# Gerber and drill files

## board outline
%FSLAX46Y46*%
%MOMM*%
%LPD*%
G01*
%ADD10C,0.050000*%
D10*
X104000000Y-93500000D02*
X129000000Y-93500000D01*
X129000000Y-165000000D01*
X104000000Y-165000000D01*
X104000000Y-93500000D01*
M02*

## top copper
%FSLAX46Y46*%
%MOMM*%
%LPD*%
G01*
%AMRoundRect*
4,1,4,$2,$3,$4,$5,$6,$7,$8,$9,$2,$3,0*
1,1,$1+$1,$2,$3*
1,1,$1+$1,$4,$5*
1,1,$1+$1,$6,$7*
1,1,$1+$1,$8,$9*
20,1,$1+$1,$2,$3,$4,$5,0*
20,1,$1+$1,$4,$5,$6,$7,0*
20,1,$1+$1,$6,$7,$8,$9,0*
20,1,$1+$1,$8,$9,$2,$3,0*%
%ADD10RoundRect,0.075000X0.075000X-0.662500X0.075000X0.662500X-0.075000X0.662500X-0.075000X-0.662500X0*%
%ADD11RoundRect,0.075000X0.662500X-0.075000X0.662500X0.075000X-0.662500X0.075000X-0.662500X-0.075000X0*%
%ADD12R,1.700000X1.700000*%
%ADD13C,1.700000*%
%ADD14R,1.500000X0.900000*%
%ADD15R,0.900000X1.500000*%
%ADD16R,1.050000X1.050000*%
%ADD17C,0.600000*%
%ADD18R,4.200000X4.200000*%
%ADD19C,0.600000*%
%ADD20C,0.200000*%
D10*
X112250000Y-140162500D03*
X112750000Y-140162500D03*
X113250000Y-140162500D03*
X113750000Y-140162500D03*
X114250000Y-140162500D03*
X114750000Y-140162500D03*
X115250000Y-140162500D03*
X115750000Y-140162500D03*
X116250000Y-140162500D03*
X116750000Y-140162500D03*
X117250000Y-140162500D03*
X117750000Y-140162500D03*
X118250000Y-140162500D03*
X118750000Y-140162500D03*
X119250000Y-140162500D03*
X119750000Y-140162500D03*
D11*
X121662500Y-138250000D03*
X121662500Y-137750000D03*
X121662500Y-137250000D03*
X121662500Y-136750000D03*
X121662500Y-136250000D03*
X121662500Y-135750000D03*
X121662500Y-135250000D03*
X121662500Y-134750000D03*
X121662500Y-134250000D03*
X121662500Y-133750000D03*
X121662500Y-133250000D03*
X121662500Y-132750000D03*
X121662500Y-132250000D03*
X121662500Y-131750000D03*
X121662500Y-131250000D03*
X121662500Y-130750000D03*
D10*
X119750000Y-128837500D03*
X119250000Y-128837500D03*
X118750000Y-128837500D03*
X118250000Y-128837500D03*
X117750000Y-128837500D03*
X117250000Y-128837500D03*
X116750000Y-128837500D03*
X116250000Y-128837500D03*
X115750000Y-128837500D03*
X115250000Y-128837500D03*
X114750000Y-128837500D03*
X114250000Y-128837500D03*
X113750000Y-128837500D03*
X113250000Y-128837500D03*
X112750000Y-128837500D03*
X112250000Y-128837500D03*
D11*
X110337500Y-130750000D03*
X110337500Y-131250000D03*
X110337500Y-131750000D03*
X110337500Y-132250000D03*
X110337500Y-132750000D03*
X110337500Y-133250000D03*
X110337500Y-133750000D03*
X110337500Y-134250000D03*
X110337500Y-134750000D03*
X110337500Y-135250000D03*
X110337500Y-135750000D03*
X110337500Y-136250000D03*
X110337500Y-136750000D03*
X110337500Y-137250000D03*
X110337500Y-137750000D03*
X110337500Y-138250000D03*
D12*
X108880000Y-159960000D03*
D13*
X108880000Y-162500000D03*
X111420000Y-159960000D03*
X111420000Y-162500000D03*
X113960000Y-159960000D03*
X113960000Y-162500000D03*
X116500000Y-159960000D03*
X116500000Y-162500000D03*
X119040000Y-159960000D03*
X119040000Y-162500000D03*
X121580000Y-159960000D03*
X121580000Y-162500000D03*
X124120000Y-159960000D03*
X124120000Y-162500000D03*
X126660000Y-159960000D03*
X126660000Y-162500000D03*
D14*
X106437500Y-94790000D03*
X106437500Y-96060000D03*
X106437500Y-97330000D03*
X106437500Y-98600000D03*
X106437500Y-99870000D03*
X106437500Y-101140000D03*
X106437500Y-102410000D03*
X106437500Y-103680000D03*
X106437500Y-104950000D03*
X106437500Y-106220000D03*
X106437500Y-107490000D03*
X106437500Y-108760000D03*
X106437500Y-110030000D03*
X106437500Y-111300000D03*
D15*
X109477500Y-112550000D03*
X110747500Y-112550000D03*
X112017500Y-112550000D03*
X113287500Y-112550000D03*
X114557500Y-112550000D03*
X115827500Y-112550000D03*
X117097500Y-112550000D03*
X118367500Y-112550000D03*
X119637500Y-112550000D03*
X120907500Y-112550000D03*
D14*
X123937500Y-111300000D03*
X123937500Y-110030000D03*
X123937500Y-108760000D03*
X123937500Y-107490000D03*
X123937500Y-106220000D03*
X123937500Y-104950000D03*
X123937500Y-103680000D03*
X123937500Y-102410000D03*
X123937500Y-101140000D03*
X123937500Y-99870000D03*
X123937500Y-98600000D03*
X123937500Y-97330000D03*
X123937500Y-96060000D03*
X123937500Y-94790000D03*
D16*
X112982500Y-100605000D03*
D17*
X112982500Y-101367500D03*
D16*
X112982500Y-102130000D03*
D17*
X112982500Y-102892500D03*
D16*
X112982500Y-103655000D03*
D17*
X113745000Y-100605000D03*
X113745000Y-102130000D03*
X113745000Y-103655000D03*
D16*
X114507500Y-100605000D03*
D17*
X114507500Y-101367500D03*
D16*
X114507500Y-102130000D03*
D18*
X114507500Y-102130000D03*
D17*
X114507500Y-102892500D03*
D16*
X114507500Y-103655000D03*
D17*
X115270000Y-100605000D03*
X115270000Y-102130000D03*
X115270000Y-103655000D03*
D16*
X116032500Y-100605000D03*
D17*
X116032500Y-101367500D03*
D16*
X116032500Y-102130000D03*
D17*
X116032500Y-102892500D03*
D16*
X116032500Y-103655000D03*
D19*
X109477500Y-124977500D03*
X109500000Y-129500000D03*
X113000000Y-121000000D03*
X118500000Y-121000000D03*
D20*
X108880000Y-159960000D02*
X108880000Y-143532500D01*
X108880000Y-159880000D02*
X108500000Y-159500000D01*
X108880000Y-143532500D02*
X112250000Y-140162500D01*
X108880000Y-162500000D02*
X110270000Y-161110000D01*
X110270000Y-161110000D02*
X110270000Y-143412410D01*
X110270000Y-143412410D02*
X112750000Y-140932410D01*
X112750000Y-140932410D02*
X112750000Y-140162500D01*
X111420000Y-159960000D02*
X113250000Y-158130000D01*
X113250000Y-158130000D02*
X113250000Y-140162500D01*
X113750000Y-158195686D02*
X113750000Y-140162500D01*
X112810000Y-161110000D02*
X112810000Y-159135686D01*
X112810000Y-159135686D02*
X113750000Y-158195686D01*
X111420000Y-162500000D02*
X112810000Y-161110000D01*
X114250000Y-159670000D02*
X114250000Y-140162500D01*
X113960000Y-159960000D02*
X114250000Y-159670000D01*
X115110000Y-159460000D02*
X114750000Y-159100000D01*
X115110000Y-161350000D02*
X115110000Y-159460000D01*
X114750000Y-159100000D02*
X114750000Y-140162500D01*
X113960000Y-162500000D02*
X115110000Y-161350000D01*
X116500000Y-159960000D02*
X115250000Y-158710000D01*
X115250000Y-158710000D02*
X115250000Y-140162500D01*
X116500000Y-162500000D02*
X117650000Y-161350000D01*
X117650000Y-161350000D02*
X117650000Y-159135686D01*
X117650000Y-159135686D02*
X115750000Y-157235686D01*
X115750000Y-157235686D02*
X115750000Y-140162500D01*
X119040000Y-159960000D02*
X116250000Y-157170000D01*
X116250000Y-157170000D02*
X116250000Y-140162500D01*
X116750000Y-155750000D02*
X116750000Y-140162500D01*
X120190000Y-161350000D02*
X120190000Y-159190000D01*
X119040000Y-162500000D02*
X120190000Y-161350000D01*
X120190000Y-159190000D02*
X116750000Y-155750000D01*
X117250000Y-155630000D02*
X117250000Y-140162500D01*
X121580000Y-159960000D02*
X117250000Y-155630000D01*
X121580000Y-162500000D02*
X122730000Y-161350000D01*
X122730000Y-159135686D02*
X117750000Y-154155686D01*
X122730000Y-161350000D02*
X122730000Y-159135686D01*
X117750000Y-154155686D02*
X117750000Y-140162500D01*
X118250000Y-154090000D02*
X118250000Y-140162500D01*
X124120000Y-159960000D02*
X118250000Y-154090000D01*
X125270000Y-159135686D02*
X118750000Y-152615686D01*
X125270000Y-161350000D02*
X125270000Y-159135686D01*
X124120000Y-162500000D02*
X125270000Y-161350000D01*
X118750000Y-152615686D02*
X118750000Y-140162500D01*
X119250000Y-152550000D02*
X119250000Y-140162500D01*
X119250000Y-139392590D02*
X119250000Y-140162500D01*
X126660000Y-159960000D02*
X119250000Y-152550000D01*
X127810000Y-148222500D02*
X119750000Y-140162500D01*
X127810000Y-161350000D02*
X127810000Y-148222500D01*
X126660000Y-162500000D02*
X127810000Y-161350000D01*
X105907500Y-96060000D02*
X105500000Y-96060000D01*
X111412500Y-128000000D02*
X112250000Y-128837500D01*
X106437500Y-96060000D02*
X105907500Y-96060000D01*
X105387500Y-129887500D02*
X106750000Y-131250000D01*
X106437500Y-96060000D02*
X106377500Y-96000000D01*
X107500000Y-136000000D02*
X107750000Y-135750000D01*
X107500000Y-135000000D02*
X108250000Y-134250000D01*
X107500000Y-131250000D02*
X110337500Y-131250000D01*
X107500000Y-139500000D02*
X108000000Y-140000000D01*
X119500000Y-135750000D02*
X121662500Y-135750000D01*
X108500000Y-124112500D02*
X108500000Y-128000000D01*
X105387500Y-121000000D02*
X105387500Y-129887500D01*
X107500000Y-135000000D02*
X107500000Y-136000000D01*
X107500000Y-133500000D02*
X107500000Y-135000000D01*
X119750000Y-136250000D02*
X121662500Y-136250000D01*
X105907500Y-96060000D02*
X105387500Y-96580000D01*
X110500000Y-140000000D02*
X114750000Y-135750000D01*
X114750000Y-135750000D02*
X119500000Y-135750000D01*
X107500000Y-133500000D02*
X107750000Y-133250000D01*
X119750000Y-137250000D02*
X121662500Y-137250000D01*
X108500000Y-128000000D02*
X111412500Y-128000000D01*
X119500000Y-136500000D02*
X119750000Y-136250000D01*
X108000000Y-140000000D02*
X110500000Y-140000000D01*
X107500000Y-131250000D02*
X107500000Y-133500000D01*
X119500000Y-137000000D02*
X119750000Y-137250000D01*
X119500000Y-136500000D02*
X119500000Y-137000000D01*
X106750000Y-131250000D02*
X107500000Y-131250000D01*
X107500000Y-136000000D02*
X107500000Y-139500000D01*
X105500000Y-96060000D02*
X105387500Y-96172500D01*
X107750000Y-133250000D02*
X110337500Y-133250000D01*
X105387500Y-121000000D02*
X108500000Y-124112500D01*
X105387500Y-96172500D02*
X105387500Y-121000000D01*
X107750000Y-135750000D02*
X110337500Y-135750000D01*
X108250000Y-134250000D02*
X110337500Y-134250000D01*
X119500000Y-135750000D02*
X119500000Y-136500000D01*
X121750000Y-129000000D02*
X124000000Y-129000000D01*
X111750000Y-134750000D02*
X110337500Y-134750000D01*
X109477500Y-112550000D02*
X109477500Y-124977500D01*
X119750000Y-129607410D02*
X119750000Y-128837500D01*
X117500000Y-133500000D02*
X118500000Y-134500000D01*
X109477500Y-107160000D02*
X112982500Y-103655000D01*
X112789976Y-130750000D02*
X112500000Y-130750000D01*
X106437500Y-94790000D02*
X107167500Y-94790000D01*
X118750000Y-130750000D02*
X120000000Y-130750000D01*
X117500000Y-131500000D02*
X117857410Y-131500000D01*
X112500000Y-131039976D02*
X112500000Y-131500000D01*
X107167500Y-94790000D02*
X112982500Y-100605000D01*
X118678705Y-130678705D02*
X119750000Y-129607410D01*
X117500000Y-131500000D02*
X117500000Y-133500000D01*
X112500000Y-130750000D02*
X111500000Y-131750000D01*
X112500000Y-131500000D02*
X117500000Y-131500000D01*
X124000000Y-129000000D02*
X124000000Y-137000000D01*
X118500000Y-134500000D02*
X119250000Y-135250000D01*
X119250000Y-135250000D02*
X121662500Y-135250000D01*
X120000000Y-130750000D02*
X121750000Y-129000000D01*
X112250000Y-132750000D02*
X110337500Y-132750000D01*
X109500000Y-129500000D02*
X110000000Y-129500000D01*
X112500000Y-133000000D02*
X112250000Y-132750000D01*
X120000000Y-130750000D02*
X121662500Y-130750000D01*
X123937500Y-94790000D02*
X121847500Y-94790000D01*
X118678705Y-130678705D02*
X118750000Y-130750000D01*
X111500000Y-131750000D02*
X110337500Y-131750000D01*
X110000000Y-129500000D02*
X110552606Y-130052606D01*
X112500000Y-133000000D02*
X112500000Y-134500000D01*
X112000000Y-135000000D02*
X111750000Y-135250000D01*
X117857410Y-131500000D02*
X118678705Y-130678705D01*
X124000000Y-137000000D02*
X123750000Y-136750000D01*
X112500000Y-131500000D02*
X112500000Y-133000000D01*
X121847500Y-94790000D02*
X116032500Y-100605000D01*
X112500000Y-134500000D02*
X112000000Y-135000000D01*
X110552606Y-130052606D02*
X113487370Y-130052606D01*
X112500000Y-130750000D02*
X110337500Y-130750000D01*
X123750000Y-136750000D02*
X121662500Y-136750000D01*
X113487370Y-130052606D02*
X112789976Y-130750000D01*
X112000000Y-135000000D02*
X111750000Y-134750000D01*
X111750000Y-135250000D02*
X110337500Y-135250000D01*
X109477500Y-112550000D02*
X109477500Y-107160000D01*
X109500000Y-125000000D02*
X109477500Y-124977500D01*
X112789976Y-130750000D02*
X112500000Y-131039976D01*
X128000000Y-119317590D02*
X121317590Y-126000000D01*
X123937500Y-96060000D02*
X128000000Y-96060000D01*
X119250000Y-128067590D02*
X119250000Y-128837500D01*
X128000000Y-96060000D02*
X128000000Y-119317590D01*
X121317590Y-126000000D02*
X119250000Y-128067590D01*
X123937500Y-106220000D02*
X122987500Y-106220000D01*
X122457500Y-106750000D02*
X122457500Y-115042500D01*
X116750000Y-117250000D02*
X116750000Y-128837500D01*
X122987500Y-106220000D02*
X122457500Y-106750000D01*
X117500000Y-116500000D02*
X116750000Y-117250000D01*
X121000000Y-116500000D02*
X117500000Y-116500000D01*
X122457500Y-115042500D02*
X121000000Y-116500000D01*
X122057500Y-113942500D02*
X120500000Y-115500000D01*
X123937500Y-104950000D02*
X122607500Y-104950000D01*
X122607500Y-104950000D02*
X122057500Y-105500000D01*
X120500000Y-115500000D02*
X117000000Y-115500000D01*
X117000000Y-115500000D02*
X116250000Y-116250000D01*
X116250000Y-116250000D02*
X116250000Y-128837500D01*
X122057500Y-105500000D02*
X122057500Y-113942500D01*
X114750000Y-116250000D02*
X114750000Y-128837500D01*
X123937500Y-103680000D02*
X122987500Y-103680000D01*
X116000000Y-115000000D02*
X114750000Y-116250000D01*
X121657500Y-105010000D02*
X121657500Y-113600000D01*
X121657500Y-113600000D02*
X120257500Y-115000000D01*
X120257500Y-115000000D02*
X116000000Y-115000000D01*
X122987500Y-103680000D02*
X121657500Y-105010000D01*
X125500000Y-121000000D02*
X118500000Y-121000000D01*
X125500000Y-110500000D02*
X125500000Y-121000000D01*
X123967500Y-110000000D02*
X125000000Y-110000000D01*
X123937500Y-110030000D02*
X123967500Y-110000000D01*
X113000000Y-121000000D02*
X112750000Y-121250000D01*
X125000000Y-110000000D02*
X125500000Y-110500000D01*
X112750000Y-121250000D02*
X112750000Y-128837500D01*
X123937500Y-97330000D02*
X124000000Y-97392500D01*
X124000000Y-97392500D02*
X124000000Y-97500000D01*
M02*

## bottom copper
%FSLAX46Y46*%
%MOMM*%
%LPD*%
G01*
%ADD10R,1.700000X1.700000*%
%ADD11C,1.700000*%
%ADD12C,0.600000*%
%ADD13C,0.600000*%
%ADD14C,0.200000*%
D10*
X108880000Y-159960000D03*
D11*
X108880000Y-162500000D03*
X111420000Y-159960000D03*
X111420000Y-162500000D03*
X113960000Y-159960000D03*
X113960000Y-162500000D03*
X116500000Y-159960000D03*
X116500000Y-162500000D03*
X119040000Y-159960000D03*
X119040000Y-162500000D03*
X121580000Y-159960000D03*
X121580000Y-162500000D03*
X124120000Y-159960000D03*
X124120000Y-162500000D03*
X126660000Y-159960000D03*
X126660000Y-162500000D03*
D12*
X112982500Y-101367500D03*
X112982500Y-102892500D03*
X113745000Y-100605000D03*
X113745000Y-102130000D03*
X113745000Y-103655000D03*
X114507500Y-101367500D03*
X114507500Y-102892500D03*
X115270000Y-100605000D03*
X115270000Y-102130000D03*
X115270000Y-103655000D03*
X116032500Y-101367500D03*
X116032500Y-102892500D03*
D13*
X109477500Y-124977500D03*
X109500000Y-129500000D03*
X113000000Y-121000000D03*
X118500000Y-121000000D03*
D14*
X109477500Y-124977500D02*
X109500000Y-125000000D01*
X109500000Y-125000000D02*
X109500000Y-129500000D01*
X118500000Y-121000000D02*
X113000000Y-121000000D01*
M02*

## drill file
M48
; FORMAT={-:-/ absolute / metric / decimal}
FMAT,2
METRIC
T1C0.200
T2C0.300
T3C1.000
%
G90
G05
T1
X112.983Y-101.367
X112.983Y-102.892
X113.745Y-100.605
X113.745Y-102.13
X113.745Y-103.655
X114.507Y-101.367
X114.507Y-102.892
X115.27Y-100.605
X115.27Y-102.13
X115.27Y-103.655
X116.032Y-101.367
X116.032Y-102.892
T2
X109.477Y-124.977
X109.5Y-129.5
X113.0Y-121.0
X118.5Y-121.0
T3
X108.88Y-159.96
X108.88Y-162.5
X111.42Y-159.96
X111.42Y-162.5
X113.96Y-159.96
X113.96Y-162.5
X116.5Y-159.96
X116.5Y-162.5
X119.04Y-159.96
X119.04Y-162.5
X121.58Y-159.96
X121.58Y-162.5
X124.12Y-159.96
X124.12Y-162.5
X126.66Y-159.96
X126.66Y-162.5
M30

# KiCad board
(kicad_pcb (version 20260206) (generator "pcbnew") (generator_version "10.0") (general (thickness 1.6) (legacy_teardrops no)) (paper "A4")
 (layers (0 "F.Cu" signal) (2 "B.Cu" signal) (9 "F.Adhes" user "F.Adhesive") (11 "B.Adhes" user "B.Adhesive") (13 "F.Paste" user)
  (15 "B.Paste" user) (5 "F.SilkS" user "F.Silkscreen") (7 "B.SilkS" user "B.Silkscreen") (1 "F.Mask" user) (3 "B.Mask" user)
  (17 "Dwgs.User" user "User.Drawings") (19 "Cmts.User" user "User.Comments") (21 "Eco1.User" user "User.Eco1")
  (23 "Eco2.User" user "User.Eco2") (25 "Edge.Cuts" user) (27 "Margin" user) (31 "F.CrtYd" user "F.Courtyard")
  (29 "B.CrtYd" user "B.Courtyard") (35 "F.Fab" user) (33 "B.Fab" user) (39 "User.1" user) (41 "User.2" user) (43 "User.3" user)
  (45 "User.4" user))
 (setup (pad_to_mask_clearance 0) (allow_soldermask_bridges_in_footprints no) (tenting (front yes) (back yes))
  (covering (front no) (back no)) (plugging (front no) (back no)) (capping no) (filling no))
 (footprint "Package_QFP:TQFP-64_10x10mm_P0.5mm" (layer "F.Cu") (at 116 134.5 90)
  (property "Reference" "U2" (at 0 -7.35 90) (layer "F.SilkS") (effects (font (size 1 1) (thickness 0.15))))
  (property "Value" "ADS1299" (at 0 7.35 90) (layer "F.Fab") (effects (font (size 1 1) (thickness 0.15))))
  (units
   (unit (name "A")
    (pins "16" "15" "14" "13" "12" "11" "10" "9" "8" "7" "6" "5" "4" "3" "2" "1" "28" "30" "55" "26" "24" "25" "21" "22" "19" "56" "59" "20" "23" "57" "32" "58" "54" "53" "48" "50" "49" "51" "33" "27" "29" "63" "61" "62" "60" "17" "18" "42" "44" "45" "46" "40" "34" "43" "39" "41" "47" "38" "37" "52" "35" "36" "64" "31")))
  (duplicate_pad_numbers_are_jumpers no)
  (pad "1" smd roundrect (at -5.6625 -3.75 90) (size 1.475 0.3) (layers "F.Cu" "F.Mask" "F.Paste") (roundrect_rratio 0.25)
   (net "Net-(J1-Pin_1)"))
  (pad "2" smd roundrect (at -5.6625 -3.25 90) (size 1.475 0.3) (layers "F.Cu" "F.Mask" "F.Paste") (roundrect_rratio 0.25)
   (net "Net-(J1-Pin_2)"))
  (pad "3" smd roundrect (at -5.6625 -2.75 90) (size 1.475 0.3) (layers "F.Cu" "F.Mask" "F.Paste") (roundrect_rratio 0.25)
   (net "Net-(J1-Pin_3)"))
  (pad "4" smd roundrect (at -5.6625 -2.25 90) (size 1.475 0.3) (layers "F.Cu" "F.Mask" "F.Paste") (roundrect_rratio 0.25)
   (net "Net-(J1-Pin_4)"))
  (pad "5" smd roundrect (at -5.6625 -1.75 90) (size 1.475 0.3) (layers "F.Cu" "F.Mask" "F.Paste") (roundrect_rratio 0.25)
   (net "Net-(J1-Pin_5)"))
  (pad "6" smd roundrect (at -5.6625 -1.25 90) (size 1.475 0.3) (layers "F.Cu" "F.Mask" "F.Paste") (roundrect_rratio 0.25)
   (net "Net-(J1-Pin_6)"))
  (pad "7" smd roundrect (at -5.6625 -0.75 90) (size 1.475 0.3) (layers "F.Cu" "F.Mask" "F.Paste") (roundrect_rratio 0.25)
   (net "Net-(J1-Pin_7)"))
  (pad "8" smd roundrect (at -5.6625 -0.25 90) (size 1.475 0.3) (layers "F.Cu" "F.Mask" "F.Paste") (roundrect_rratio 0.25)
   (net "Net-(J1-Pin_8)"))
  (pad "9" smd roundrect (at -5.6625 0.25 90) (size 1.475 0.3) (layers "F.Cu" "F.Mask" "F.Paste") (roundrect_rratio 0.25)
   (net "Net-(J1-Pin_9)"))
  (pad "10" smd roundrect (at -5.6625 0.75 90) (size 1.475 0.3) (layers "F.Cu" "F.Mask" "F.Paste") (roundrect_rratio 0.25)
   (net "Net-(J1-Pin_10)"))
  (pad "11" smd roundrect (at -5.6625 1.25 90) (size 1.475 0.3) (layers "F.Cu" "F.Mask" "F.Paste") (roundrect_rratio 0.25)
   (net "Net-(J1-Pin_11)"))
  (pad "12" smd roundrect (at -5.6625 1.75 90) (size 1.475 0.3) (layers "F.Cu" "F.Mask" "F.Paste") (roundrect_rratio 0.25)
   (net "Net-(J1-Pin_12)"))
  (pad "13" smd roundrect (at -5.6625 2.25 90) (size 1.475 0.3) (layers "F.Cu" "F.Mask" "F.Paste") (roundrect_rratio 0.25)
   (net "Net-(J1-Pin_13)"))
  (pad "14" smd roundrect (at -5.6625 2.75 90) (size 1.475 0.3) (layers "F.Cu" "F.Mask" "F.Paste") (roundrect_rratio 0.25)
   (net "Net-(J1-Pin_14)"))
  (pad "15" smd roundrect (at -5.6625 3.25 90) (size 1.475 0.3) (layers "F.Cu" "F.Mask" "F.Paste") (roundrect_rratio 0.25)
   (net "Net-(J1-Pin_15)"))
  (pad "16" smd roundrect (at -5.6625 3.75 90) (size 1.475 0.3) (layers "F.Cu" "F.Mask" "F.Paste") (roundrect_rratio 0.25)
   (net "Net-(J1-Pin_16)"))
  (pad "17" smd roundrect (at -3.75 5.6625 90) (size 0.3 1.475) (layers "F.Cu" "F.Mask" "F.Paste") (roundrect_rratio 0.25)
   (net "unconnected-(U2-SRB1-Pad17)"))
  (pad "18" smd roundrect (at -3.25 5.6625 90) (size 0.3 1.475) (layers "F.Cu" "F.Mask" "F.Paste") (roundrect_rratio 0.25)
   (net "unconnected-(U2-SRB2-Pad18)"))
  (pad "19" smd roundrect (at -2.75 5.6625 90) (size 0.3 1.475) (layers "F.Cu" "F.Mask" "F.Paste") (roundrect_rratio 0.25) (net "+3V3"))
  (pad "20" smd roundrect (at -2.25 5.6625 90) (size 0.3 1.475) (layers "F.Cu" "F.Mask" "F.Paste") (roundrect_rratio 0.25) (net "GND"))
  (pad "21" smd roundrect (at -1.75 5.6625 90) (size 0.3 1.475) (layers "F.Cu" "F.Mask" "F.Paste") (roundrect_rratio 0.25) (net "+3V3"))
  (pad "22" smd roundrect (at -1.25 5.6625 90) (size 0.3 1.475) (layers "F.Cu" "F.Mask" "F.Paste") (roundrect_rratio 0.25) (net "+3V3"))
  (pad "23" smd roundrect (at -0.75 5.6625 90) (size 0.3 1.475) (layers "F.Cu" "F.Mask" "F.Paste") (roundrect_rratio 0.25) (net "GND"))
  (pad "24" smd roundrect (at -0.25 5.6625 90) (size 0.3 1.475) (layers "F.Cu" "F.Mask" "F.Paste") (roundrect_rratio 0.25)
   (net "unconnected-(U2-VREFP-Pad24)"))
  (pad "25" smd roundrect (at 0.25 5.6625 90) (size 0.3 1.475) (layers "F.Cu" "F.Mask" "F.Paste") (roundrect_rratio 0.25)
   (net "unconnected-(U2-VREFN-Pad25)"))
  (pad "26" smd roundrect (at 0.75 5.6625 90) (size 0.3 1.475) (layers "F.Cu" "F.Mask" "F.Paste") (roundrect_rratio 0.25)
   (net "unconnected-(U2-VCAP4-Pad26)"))
  (pad "27" smd roundrect (at 1.25 5.6625 90) (size 0.3 1.475) (layers "F.Cu" "F.Mask" "F.Paste") (roundrect_rratio 0.25)
   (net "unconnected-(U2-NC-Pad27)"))
  (pad "28" smd roundrect (at 1.75 5.6625 90) (size 0.3 1.475) (layers "F.Cu" "F.Mask" "F.Paste") (roundrect_rratio 0.25)
   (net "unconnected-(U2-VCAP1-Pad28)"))
  (pad "29" smd roundrect (at 2.25 5.6625 90) (size 0.3 1.475) (layers "F.Cu" "F.Mask" "F.Paste") (roundrect_rratio 0.25)
   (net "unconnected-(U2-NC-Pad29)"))
  (pad "30" smd roundrect (at 2.75 5.6625 90) (size 0.3 1.475) (layers "F.Cu" "F.Mask" "F.Paste") (roundrect_rratio 0.25)
   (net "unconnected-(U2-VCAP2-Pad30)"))
  (pad "31" smd roundrect (at 3.25 5.6625 90) (size 0.3 1.475) (layers "F.Cu" "F.Mask" "F.Paste") (roundrect_rratio 0.25)
   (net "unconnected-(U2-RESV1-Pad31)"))
  (pad "32" smd roundrect (at 3.75 5.6625 90) (size 0.3 1.475) (layers "F.Cu" "F.Mask" "F.Paste") (roundrect_rratio 0.25) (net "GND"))
  (pad "33" smd roundrect (at 5.6625 3.75 90) (size 1.475 0.3) (layers "F.Cu" "F.Mask" "F.Paste") (roundrect_rratio 0.25) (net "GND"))
  (pad "34" smd roundrect (at 5.6625 3.25 90) (size 1.475 0.3) (layers "F.Cu" "F.Mask" "F.Paste") (roundrect_rratio 0.25)
   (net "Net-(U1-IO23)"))
  (pad "35" smd roundrect (at 5.6625 2.75 90) (size 1.475 0.3) (layers "F.Cu" "F.Mask" "F.Paste") (roundrect_rratio 0.25)
   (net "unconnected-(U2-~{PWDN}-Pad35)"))
  (pad "36" smd roundrect (at 5.6625 2.25 90) (size 1.475 0.3) (layers "F.Cu" "F.Mask" "F.Paste") (roundrect_rratio 0.25)
   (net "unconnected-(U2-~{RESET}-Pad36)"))
  (pad "37" smd roundrect (at 5.6625 1.75 90) (size 1.475 0.3) (layers "F.Cu" "F.Mask" "F.Paste") (roundrect_rratio 0.25)
   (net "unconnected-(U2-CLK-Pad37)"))
  (pad "38" smd roundrect (at 5.6625 1.25 90) (size 1.475 0.3) (layers "F.Cu" "F.Mask" "F.Paste") (roundrect_rratio 0.25)
   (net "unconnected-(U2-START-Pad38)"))
  (pad "39" smd roundrect (at 5.6625 0.75 90) (size 1.475 0.3) (layers "F.Cu" "F.Mask" "F.Paste") (roundrect_rratio 0.25)
   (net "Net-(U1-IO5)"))
  (pad "40" smd roundrect (at 5.6625 0.25 90) (size 1.475 0.3) (layers "F.Cu" "F.Mask" "F.Paste") (roundrect_rratio 0.25)
   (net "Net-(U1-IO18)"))
  (pad "41" smd roundrect (at 5.6625 -0.25 90) (size 1.475 0.3) (layers "F.Cu" "F.Mask" "F.Paste") (roundrect_rratio 0.25)
   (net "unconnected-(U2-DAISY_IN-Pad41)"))
  (pad "42" smd roundrect (at 5.6625 -0.75 90) (size 1.475 0.3) (layers "F.Cu" "F.Mask" "F.Paste") (roundrect_rratio 0.25)
   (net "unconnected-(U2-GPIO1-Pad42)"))
  (pad "43" smd roundrect (at 5.6625 -1.25 90) (size 1.475 0.3) (layers "F.Cu" "F.Mask" "F.Paste") (roundrect_rratio 0.25)
   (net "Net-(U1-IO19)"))
  (pad "44" smd roundrect (at 5.6625 -1.75 90) (size 1.475 0.3) (layers "F.Cu" "F.Mask" "F.Paste") (roundrect_rratio 0.25)
   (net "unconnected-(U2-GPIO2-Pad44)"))
  (pad "45" smd roundrect (at 5.6625 -2.25 90) (size 1.475 0.3) (layers "F.Cu" "F.Mask" "F.Paste") (roundrect_rratio 0.25)
   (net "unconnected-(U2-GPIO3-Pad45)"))
  (pad "46" smd roundrect (at 5.6625 -2.75 90) (size 1.475 0.3) (layers "F.Cu" "F.Mask" "F.Paste") (roundrect_rratio 0.25)
   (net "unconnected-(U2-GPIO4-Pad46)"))
  (pad "47" smd roundrect (at 5.6625 -3.25 90) (size 1.475 0.3) (layers "F.Cu" "F.Mask" "F.Paste") (roundrect_rratio 0.25)
   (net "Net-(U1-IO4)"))
  (pad "48" smd roundrect (at 5.6625 -3.75 90) (size 1.475 0.3) (layers "F.Cu" "F.Mask" "F.Paste") (roundrect_rratio 0.25) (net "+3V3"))
  (pad "49" smd roundrect (at 3.75 -5.6625 90) (size 0.3 1.475) (layers "F.Cu" "F.Mask" "F.Paste") (roundrect_rratio 0.25) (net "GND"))
  (pad "50" smd roundrect (at 3.25 -5.6625 90) (size 0.3 1.475) (layers "F.Cu" "F.Mask" "F.Paste") (roundrect_rratio 0.25) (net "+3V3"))
  (pad "51" smd roundrect (at 2.75 -5.6625 90) (size 0.3 1.475) (layers "F.Cu" "F.Mask" "F.Paste") (roundrect_rratio 0.25) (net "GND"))
  (pad "52" smd roundrect (at 2.25 -5.6625 90) (size 0.3 1.475) (layers "F.Cu" "F.Mask" "F.Paste") (roundrect_rratio 0.25)
   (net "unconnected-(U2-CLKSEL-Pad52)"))
  (pad "53" smd roundrect (at 1.75 -5.6625 90) (size 0.3 1.475) (layers "F.Cu" "F.Mask" "F.Paste") (roundrect_rratio 0.25) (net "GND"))
  (pad "54" smd roundrect (at 1.25 -5.6625 90) (size 0.3 1.475) (layers "F.Cu" "F.Mask" "F.Paste") (roundrect_rratio 0.25) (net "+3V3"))
  (pad "55" smd roundrect (at 0.75 -5.6625 90) (size 0.3 1.475) (layers "F.Cu" "F.Mask" "F.Paste") (roundrect_rratio 0.25)
   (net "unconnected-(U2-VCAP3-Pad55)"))
  (pad "56" smd roundrect (at 0.25 -5.6625 90) (size 0.3 1.475) (layers "F.Cu" "F.Mask" "F.Paste") (roundrect_rratio 0.25) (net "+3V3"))
  (pad "57" smd roundrect (at -0.25 -5.6625 90) (size 0.3 1.475) (layers "F.Cu" "F.Mask" "F.Paste") (roundrect_rratio 0.25) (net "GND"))
  (pad "58" smd roundrect (at -0.75 -5.6625 90) (size 0.3 1.475) (layers "F.Cu" "F.Mask" "F.Paste") (roundrect_rratio 0.25) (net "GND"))
  (pad "59" smd roundrect (at -1.25 -5.6625 90) (size 0.3 1.475) (layers "F.Cu" "F.Mask" "F.Paste") (roundrect_rratio 0.25) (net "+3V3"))
  (pad "60" smd roundrect (at -1.75 -5.6625 90) (size 0.3 1.475) (layers "F.Cu" "F.Mask" "F.Paste") (roundrect_rratio 0.25)
   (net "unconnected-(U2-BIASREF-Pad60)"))
  (pad "61" smd roundrect (at -2.25 -5.6625 90) (size 0.3 1.475) (layers "F.Cu" "F.Mask" "F.Paste") (roundrect_rratio 0.25)
   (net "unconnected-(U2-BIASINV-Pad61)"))
  (pad "62" smd roundrect (at -2.75 -5.6625 90) (size 0.3 1.475) (layers "F.Cu" "F.Mask" "F.Paste") (roundrect_rratio 0.25)
   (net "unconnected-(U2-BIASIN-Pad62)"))
  (pad "63" smd roundrect (at -3.25 -5.6625 90) (size 0.3 1.475) (layers "F.Cu" "F.Mask" "F.Paste") (roundrect_rratio 0.25)
   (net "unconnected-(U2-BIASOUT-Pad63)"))
  (pad "64" smd roundrect (at -3.75 -5.6625 90) (size 0.3 1.475) (layers "F.Cu" "F.Mask" "F.Paste") (roundrect_rratio 0.25)
   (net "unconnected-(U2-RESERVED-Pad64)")))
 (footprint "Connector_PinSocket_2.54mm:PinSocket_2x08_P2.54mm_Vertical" (layer "F.Cu") (at 108.88 159.96 90)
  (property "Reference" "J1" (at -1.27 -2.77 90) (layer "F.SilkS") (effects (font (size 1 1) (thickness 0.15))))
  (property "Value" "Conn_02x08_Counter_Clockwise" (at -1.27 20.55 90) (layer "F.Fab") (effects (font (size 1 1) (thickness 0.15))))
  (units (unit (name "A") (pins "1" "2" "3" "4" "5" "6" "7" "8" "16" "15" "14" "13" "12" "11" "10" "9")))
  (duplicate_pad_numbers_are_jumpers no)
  (pad "1" thru_hole rect (at 0 0 90) (size 1.7 1.7) (drill 1) (layers "*.Cu" "*.Mask") (remove_unused_layers no) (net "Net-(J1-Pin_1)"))
  (pad "2" thru_hole circle (at -2.54 0 90) (size 1.7 1.7) (drill 1) (layers "*.Cu" "*.Mask") (remove_unused_layers no)
   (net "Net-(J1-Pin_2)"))
  (pad "3" thru_hole circle (at 0 2.54 90) (size 1.7 1.7) (drill 1) (layers "*.Cu" "*.Mask") (remove_unused_layers no)
   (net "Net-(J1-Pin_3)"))
  (pad "4" thru_hole circle (at -2.54 2.54 90) (size 1.7 1.7) (drill 1) (layers "*.Cu" "*.Mask") (remove_unused_layers no)
   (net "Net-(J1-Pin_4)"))
  (pad "5" thru_hole circle (at 0 5.08 90) (size 1.7 1.7) (drill 1) (layers "*.Cu" "*.Mask") (remove_unused_layers no)
   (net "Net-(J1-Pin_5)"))
  (pad "6" thru_hole circle (at -2.54 5.08 90) (size 1.7 1.7) (drill 1) (layers "*.Cu" "*.Mask") (remove_unused_layers no)
   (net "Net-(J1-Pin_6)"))
  (pad "7" thru_hole circle (at 0 7.62 90) (size 1.7 1.7) (drill 1) (layers "*.Cu" "*.Mask") (remove_unused_layers no)
   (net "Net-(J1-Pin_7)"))
  (pad "8" thru_hole circle (at -2.54 7.62 90) (size 1.7 1.7) (drill 1) (layers "*.Cu" "*.Mask") (remove_unused_layers no)
   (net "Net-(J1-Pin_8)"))
  (pad "9" thru_hole circle (at 0 10.16 90) (size 1.7 1.7) (drill 1) (layers "*.Cu" "*.Mask") (remove_unused_layers no)
   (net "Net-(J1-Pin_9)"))
  (pad "10" thru_hole circle (at -2.54 10.16 90) (size 1.7 1.7) (drill 1) (layers "*.Cu" "*.Mask") (remove_unused_layers no)
   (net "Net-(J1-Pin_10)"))
  (pad "11" thru_hole circle (at 0 12.7 90) (size 1.7 1.7) (drill 1) (layers "*.Cu" "*.Mask") (remove_unused_layers no)
   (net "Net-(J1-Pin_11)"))
  (pad "12" thru_hole circle (at -2.54 12.7 90) (size 1.7 1.7) (drill 1) (layers "*.Cu" "*.Mask") (remove_unused_layers no)
   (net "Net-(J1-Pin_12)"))
  (pad "13" thru_hole circle (at 0 15.24 90) (size 1.7 1.7) (drill 1) (layers "*.Cu" "*.Mask") (remove_unused_layers no)
   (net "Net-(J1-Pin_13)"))
  (pad "14" thru_hole circle (at -2.54 15.24 90) (size 1.7 1.7) (drill 1) (layers "*.Cu" "*.Mask") (remove_unused_layers no)
   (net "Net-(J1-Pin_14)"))
  (pad "15" thru_hole circle (at 0 17.78 90) (size 1.7 1.7) (drill 1) (layers "*.Cu" "*.Mask") (remove_unused_layers no)
   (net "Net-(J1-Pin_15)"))
  (pad "16" thru_hole circle (at -2.54 17.78 90) (size 1.7 1.7) (drill 1) (layers "*.Cu" "*.Mask") (remove_unused_layers no)
   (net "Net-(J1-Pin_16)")))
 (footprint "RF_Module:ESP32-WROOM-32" (layer "F.Cu") (at 115.1875 103.04)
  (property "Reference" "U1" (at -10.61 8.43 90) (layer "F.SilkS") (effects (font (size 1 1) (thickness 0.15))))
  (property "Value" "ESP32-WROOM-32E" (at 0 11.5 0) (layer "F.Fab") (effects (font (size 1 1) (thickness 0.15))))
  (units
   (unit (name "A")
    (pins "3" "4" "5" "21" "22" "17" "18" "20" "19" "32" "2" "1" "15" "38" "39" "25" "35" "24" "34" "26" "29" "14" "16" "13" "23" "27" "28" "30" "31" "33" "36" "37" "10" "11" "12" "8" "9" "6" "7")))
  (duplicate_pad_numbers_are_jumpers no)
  (pad "1" smd rect (at -8.75 -8.25) (size 1.5 0.9) (layers "F.Cu" "F.Mask" "F.Paste") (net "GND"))
  (pad "2" smd rect (at -8.75 -6.98) (size 1.5 0.9) (layers "F.Cu" "F.Mask" "F.Paste") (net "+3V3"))
  (pad "3" smd rect (at -8.75 -5.71) (size 1.5 0.9) (layers "F.Cu" "F.Mask" "F.Paste") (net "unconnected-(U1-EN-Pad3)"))
  (pad "4" smd rect (at -8.75 -4.44) (size 1.5 0.9) (layers "F.Cu" "F.Mask" "F.Paste") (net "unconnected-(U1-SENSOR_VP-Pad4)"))
  (pad "5" smd rect (at -8.75 -3.17) (size 1.5 0.9) (layers "F.Cu" "F.Mask" "F.Paste") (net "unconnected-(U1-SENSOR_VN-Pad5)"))
  (pad "6" smd rect (at -8.75 -1.9) (size 1.5 0.9) (layers "F.Cu" "F.Mask" "F.Paste") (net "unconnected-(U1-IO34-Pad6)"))
  (pad "7" smd rect (at -8.75 -0.63) (size 1.5 0.9) (layers "F.Cu" "F.Mask" "F.Paste") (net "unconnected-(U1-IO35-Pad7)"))
  (pad "8" smd rect (at -8.75 0.64) (size 1.5 0.9) (layers "F.Cu" "F.Mask" "F.Paste") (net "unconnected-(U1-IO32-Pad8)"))
  (pad "9" smd rect (at -8.75 1.91) (size 1.5 0.9) (layers "F.Cu" "F.Mask" "F.Paste") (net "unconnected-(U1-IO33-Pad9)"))
  (pad "10" smd rect (at -8.75 3.18) (size 1.5 0.9) (layers "F.Cu" "F.Mask" "F.Paste") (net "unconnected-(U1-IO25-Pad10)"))
  (pad "11" smd rect (at -8.75 4.45) (size 1.5 0.9) (layers "F.Cu" "F.Mask" "F.Paste") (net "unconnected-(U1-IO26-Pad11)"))
  (pad "12" smd rect (at -8.75 5.72) (size 1.5 0.9) (layers "F.Cu" "F.Mask" "F.Paste") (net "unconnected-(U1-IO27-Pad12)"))
  (pad "13" smd rect (at -8.75 6.99) (size 1.5 0.9) (layers "F.Cu" "F.Mask" "F.Paste") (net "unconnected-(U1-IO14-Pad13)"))
  (pad "14" smd rect (at -8.75 8.26) (size 1.5 0.9) (layers "F.Cu" "F.Mask" "F.Paste") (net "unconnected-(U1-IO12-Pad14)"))
  (pad "15" smd rect (at -5.71 9.51 90) (size 1.5 0.9) (layers "F.Cu" "F.Mask" "F.Paste") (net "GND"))
  (pad "16" smd rect (at -4.44 9.51 90) (size 1.5 0.9) (layers "F.Cu" "F.Mask" "F.Paste") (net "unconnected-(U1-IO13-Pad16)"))
  (pad "17" smd rect (at -3.17 9.51 90) (size 1.5 0.9) (layers "F.Cu" "F.Mask" "F.Paste") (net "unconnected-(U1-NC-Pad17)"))
  (pad "18" smd rect (at -1.9 9.51 90) (size 1.5 0.9) (layers "F.Cu" "F.Mask" "F.Paste") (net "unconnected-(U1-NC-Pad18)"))
  (pad "19" smd rect (at -0.63 9.51 90) (size 1.5 0.9) (layers "F.Cu" "F.Mask" "F.Paste") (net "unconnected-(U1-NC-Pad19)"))
  (pad "20" smd rect (at 0.64 9.51 90) (size 1.5 0.9) (layers "F.Cu" "F.Mask" "F.Paste") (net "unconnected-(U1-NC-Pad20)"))
  (pad "21" smd rect (at 1.91 9.51 90) (size 1.5 0.9) (layers "F.Cu" "F.Mask" "F.Paste") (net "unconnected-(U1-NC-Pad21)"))
  (pad "22" smd rect (at 3.18 9.51 90) (size 1.5 0.9) (layers "F.Cu" "F.Mask" "F.Paste") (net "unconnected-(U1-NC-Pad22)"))
  (pad "23" smd rect (at 4.45 9.51 90) (size 1.5 0.9) (layers "F.Cu" "F.Mask" "F.Paste") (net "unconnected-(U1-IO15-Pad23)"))
  (pad "24" smd rect (at 5.72 9.51 90) (size 1.5 0.9) (layers "F.Cu" "F.Mask" "F.Paste") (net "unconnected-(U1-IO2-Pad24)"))
  (pad "25" smd rect (at 8.75 8.26) (size 1.5 0.9) (layers "F.Cu" "F.Mask" "F.Paste") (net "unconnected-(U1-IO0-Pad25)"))
  (pad "26" smd rect (at 8.75 6.99) (size 1.5 0.9) (layers "F.Cu" "F.Mask" "F.Paste") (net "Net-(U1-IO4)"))
  (pad "27" smd rect (at 8.75 5.72) (size 1.5 0.9) (layers "F.Cu" "F.Mask" "F.Paste") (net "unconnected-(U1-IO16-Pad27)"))
  (pad "28" smd rect (at 8.75 4.45) (size 1.5 0.9) (layers "F.Cu" "F.Mask" "F.Paste") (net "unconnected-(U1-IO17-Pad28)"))
  (pad "29" smd rect (at 8.75 3.18) (size 1.5 0.9) (layers "F.Cu" "F.Mask" "F.Paste") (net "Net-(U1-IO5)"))
  (pad "30" smd rect (at 8.75 1.91) (size 1.5 0.9) (layers "F.Cu" "F.Mask" "F.Paste") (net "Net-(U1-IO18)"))
  (pad "31" smd rect (at 8.75 0.64) (size 1.5 0.9) (layers "F.Cu" "F.Mask" "F.Paste") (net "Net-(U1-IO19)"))
  (pad "32" smd rect (at 8.75 -0.63) (size 1.5 0.9) (layers "F.Cu" "F.Mask" "F.Paste") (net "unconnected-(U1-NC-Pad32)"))
  (pad "33" smd rect (at 8.75 -1.9) (size 1.5 0.9) (layers "F.Cu" "F.Mask" "F.Paste") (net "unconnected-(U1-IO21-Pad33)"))
  (pad "34" smd rect (at 8.75 -3.17) (size 1.5 0.9) (layers "F.Cu" "F.Mask" "F.Paste") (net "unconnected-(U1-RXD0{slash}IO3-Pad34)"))
  (pad "35" smd rect (at 8.75 -4.44) (size 1.5 0.9) (layers "F.Cu" "F.Mask" "F.Paste") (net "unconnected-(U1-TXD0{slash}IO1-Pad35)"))
  (pad "36" smd rect (at 8.75 -5.71) (size 1.5 0.9) (layers "F.Cu" "F.Mask" "F.Paste") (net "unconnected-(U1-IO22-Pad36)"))
  (pad "37" smd rect (at 8.75 -6.98) (size 1.5 0.9) (layers "F.Cu" "F.Mask" "F.Paste") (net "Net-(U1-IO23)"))
  (pad "38" smd rect (at 8.75 -8.25) (size 1.5 0.9) (layers "F.Cu" "F.Mask" "F.Paste") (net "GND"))
  (pad "39" smd rect (at -2.205 -2.435) (size 1.05 1.05) (layers "F.Cu" "F.Paste") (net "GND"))
  (pad "39" thru_hole circle (at -2.205 -1.6725) (size 0.6 0.6) (drill 0.2) (layers "*.Cu" "F.Mask") (remove_unused_layers no) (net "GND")
   (zone_connect 2))
  (pad "39" smd rect (at -2.205 -0.91) (size 1.05 1.05) (layers "F.Cu" "F.Paste") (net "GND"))
  (pad "39" thru_hole circle (at -2.205 -0.1475) (size 0.6 0.6) (drill 0.2) (layers "*.Cu" "F.Mask") (remove_unused_layers no) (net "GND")
   (zone_connect 2))
  (pad "39" smd rect (at -2.205 0.615) (size 1.05 1.05) (layers "F.Cu" "F.Paste") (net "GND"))
  (pad "39" thru_hole circle (at -1.4425 -2.435) (size 0.6 0.6) (drill 0.2) (layers "*.Cu" "F.Mask") (remove_unused_layers no) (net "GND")
   (zone_connect 2))
  (pad "39" thru_hole circle (at -1.4425 -0.91) (size 0.6 0.6) (drill 0.2) (layers "*.Cu" "F.Mask") (remove_unused_layers no) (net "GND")
   (zone_connect 2))
  (pad "39" thru_hole circle (at -1.4425 0.615) (size 0.6 0.6) (drill 0.2) (layers "*.Cu" "F.Mask") (remove_unused_layers no) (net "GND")
   (zone_connect 2))
  (pad "39" smd rect (at -0.68 -2.435) (size 1.05 1.05) (layers "F.Cu" "F.Paste") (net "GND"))
  (pad "39" thru_hole circle (at -0.68 -1.6725) (size 0.6 0.6) (drill 0.2) (layers "*.Cu" "F.Mask") (remove_unused_layers no) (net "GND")
   (zone_connect 2))
  (pad "39" smd rect (at -0.68 -0.91) (size 1.05 1.05) (layers "F.Cu" "F.Paste") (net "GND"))
  (pad "39" smd rect (at -0.68 -0.91) (size 4.2 4.2) (layers "F.Cu" "F.Mask") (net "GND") (zone_connect 2))
  (pad "39" thru_hole circle (at -0.68 -0.1475) (size 0.6 0.6) (drill 0.2) (layers "*.Cu" "F.Mask") (remove_unused_layers no) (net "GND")
   (zone_connect 2))
  (pad "39" smd rect (at -0.68 0.615) (size 1.05 1.05) (layers "F.Cu" "F.Paste") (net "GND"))
  (pad "39" thru_hole circle (at 0.0825 -2.435) (size 0.6 0.6) (drill 0.2) (layers "*.Cu" "F.Mask") (remove_unused_layers no) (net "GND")
   (zone_connect 2))
  (pad "39" thru_hole circle (at 0.0825 -0.91) (size 0.6 0.6) (drill 0.2) (layers "*.Cu" "F.Mask") (remove_unused_layers no) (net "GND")
   (zone_connect 2))
  (pad "39" thru_hole circle (at 0.0825 0.615) (size 0.6 0.6) (drill 0.2) (layers "*.Cu" "F.Mask") (remove_unused_layers no) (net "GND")
   (zone_connect 2))
  (pad "39" smd rect (at 0.845 -2.435) (size 1.05 1.05) (layers "F.Cu" "F.Paste") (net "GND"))
  (pad "39" thru_hole circle (at 0.845 -1.6725) (size 0.6 0.6) (drill 0.2) (layers "*.Cu" "F.Mask") (remove_unused_layers no) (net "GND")
   (zone_connect 2))
  (pad "39" smd rect (at 0.845 -0.91) (size 1.05 1.05) (layers "F.Cu" "F.Paste") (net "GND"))
  (pad "39" thru_hole circle (at 0.845 -0.1475) (size 0.6 0.6) (drill 0.2) (layers "*.Cu" "F.Mask") (remove_unused_layers no) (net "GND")
   (zone_connect 2))
  (pad "39" smd rect (at 0.845 0.615) (size 1.05 1.05) (layers "F.Cu" "F.Paste") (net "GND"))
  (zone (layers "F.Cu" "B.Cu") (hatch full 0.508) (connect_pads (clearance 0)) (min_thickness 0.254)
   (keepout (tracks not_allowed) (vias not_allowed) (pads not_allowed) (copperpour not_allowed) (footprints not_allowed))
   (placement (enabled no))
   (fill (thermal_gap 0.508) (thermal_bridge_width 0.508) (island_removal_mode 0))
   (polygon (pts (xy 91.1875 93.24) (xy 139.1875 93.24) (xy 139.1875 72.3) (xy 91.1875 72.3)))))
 (gr_rect (start 104 93.5) (end 129 165) (stroke (width 0.05) (type default)) (fill no) (layer "Edge.Cuts"))
 (segment (start 108.88 159.96) (end 108.88 143.5325) (width 0.2) (layer "F.Cu") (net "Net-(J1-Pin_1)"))
 (segment (start 108.88 159.88) (end 108.5 159.5) (width 0.2) (layer "F.Cu") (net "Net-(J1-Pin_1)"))
 (segment (start 108.88 143.5325) (end 112.25 140.1625) (width 0.2) (layer "F.Cu") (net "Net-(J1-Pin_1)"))
 (segment (start 108.88 162.5) (end 110.27 161.11) (width 0.2) (layer "F.Cu") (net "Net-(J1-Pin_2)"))
 (segment (start 110.27 161.11) (end 110.27 143.41241) (width 0.2) (layer "F.Cu") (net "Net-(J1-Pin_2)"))
 (segment (start 110.27 143.41241) (end 112.75 140.93241) (width 0.2) (layer "F.Cu") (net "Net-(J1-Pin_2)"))
 (segment (start 112.75 140.93241) (end 112.75 140.1625) (width 0.2) (layer "F.Cu") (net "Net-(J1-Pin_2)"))
 (segment (start 111.42 159.96) (end 113.25 158.13) (width 0.2) (layer "F.Cu") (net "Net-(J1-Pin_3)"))
 (segment (start 113.25 158.13) (end 113.25 140.1625) (width 0.2) (layer "F.Cu") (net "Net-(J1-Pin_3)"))
 (segment (start 113.75 158.195686) (end 113.75 140.1625) (width 0.2) (layer "F.Cu") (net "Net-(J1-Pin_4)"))
 (segment (start 112.81 161.11) (end 112.81 159.135686) (width 0.2) (layer "F.Cu") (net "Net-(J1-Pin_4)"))
 (segment (start 112.81 159.135686) (end 113.75 158.195686) (width 0.2) (layer "F.Cu") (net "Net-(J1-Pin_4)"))
 (segment (start 111.42 162.5) (end 112.81 161.11) (width 0.2) (layer "F.Cu") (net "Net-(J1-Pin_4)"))
 (segment (start 114.25 159.67) (end 114.25 140.1625) (width 0.2) (layer "F.Cu") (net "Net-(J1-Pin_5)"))
 (segment (start 113.96 159.96) (end 114.25 159.67) (width 0.2) (layer "F.Cu") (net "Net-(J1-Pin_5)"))
 (segment (start 115.11 159.46) (end 114.75 159.1) (width 0.2) (layer "F.Cu") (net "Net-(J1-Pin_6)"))
 (segment (start 115.11 161.35) (end 115.11 159.46) (width 0.2) (layer "F.Cu") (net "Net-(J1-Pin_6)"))
 (segment (start 114.75 159.1) (end 114.75 140.1625) (width 0.2) (layer "F.Cu") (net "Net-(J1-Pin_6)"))
 (segment (start 113.96 162.5) (end 115.11 161.35) (width 0.2) (layer "F.Cu") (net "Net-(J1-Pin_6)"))
 (segment (start 116.5 159.96) (end 115.25 158.71) (width 0.2) (layer "F.Cu") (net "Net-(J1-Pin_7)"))
 (segment (start 115.25 158.71) (end 115.25 140.1625) (width 0.2) (layer "F.Cu") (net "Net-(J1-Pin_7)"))
 (segment (start 116.5 162.5) (end 117.65 161.35) (width 0.2) (layer "F.Cu") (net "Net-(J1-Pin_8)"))
 (segment (start 117.65 161.35) (end 117.65 159.135686) (width 0.2) (layer "F.Cu") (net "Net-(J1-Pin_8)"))
 (segment (start 117.65 159.135686) (end 115.75 157.235686) (width 0.2) (layer "F.Cu") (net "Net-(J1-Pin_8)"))
 (segment (start 115.75 157.235686) (end 115.75 140.1625) (width 0.2) (layer "F.Cu") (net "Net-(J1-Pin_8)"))
 (segment (start 119.04 159.96) (end 116.25 157.17) (width 0.2) (layer "F.Cu") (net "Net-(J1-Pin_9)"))
 (segment (start 116.25 157.17) (end 116.25 140.1625) (width 0.2) (layer "F.Cu") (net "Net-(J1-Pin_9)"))
 (segment (start 116.75 155.75) (end 116.75 140.1625) (width 0.2) (layer "F.Cu") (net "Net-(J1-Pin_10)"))
 (segment (start 120.19 161.35) (end 120.19 159.19) (width 0.2) (layer "F.Cu") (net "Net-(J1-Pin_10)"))
 (segment (start 119.04 162.5) (end 120.19 161.35) (width 0.2) (layer "F.Cu") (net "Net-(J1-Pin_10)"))
 (segment (start 120.19 159.19) (end 116.75 155.75) (width 0.2) (layer "F.Cu") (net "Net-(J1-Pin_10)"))
 (segment (start 117.25 155.63) (end 117.25 140.1625) (width 0.2) (layer "F.Cu") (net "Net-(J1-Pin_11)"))
 (segment (start 121.58 159.96) (end 117.25 155.63) (width 0.2) (layer "F.Cu") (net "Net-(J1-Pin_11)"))
 (segment (start 121.58 162.5) (end 122.73 161.35) (width 0.2) (layer "F.Cu") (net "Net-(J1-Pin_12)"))
 (segment (start 122.73 159.135686) (end 117.75 154.155686) (width 0.2) (layer "F.Cu") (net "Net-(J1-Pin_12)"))
 (segment (start 122.73 161.35) (end 122.73 159.135686) (width 0.2) (layer "F.Cu") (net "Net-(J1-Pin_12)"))
 (segment (start 117.75 154.155686) (end 117.75 140.1625) (width 0.2) (layer "F.Cu") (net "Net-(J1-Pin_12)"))
 (segment (start 118.25 154.09) (end 118.25 140.1625) (width 0.2) (layer "F.Cu") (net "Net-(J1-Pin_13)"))
 (segment (start 124.12 159.96) (end 118.25 154.09) (width 0.2) (layer "F.Cu") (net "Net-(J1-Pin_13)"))
 (segment (start 125.27 159.135686) (end 118.75 152.615686) (width 0.2) (layer "F.Cu") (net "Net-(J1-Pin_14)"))
 (segment (start 125.27 161.35) (end 125.27 159.135686) (width 0.2) (layer "F.Cu") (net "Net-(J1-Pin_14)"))
 (segment (start 124.12 162.5) (end 125.27 161.35) (width 0.2) (layer "F.Cu") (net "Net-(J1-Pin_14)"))
 (segment (start 118.75 152.615686) (end 118.75 140.1625) (width 0.2) (layer "F.Cu") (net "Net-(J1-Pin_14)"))
 (segment (start 119.25 152.55) (end 119.25 140.1625) (width 0.2) (layer "F.Cu") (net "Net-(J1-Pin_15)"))
 (segment (start 119.25 139.39259) (end 119.25 140.1625) (width 0.2) (layer "F.Cu") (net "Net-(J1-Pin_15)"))
 (segment (start 126.66 159.96) (end 119.25 152.55) (width 0.2) (layer "F.Cu") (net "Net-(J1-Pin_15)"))
 (segment (start 127.81 148.2225) (end 119.75 140.1625) (width 0.2) (layer "F.Cu") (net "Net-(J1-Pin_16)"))
 (segment (start 127.81 161.35) (end 127.81 148.2225) (width 0.2) (layer "F.Cu") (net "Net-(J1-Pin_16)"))
 (segment (start 126.66 162.5) (end 127.81 161.35) (width 0.2) (layer "F.Cu") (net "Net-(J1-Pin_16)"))
 (segment (start 105.9075 96.06) (end 105.5 96.06) (width 0.2) (layer "F.Cu") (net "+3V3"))
 (segment (start 111.4125 128) (end 112.25 128.8375) (width 0.2) (layer "F.Cu") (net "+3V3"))
 (segment (start 106.4375 96.06) (end 105.9075 96.06) (width 0.2) (layer "F.Cu") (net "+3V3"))
 (segment (start 105.3875 129.8875) (end 106.75 131.25) (width 0.2) (layer "F.Cu") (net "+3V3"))
 (segment (start 106.4375 96.06) (end 106.3775 96) (width 0.2) (layer "F.Cu") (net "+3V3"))
 (segment (start 107.5 136) (end 107.75 135.75) (width 0.2) (layer "F.Cu") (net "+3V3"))
 (segment (start 107.5 135) (end 108.25 134.25) (width 0.2) (layer "F.Cu") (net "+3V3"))
 (segment (start 107.5 131.25) (end 110.3375 131.25) (width 0.2) (layer "F.Cu") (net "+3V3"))
 (segment (start 107.5 139.5) (end 108 140) (width 0.2) (layer "F.Cu") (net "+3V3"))
 (segment (start 119.5 135.75) (end 121.6625 135.75) (width 0.2) (layer "F.Cu") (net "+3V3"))
 (segment (start 108.5 124.1125) (end 108.5 128) (width 0.2) (layer "F.Cu") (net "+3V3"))
 (segment (start 105.3875 121) (end 105.3875 129.8875) (width 0.2) (layer "F.Cu") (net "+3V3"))
 (segment (start 107.5 135) (end 107.5 136) (width 0.2) (layer "F.Cu") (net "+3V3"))
 (segment (start 107.5 133.5) (end 107.5 135) (width 0.2) (layer "F.Cu") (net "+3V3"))
 (segment (start 119.75 136.25) (end 121.6625 136.25) (width 0.2) (layer "F.Cu") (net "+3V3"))
 (segment (start 105.9075 96.06) (end 105.3875 96.58) (width 0.2) (layer "F.Cu") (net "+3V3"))
 (segment (start 110.5 140) (end 114.75 135.75) (width 0.2) (layer "F.Cu") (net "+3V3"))
 (segment (start 114.75 135.75) (end 119.5 135.75) (width 0.2) (layer "F.Cu") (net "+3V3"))
 (segment (start 107.5 133.5) (end 107.75 133.25) (width 0.2) (layer "F.Cu") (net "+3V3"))
 (segment (start 119.75 137.25) (end 121.6625 137.25) (width 0.2) (layer "F.Cu") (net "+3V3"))
 (segment (start 108.5 128) (end 111.4125 128) (width 0.2) (layer "F.Cu") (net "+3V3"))
 (segment (start 119.5 136.5) (end 119.75 136.25) (width 0.2) (layer "F.Cu") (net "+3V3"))
 (segment (start 108 140) (end 110.5 140) (width 0.2) (layer "F.Cu") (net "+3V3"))
 (segment (start 107.5 131.25) (end 107.5 133.5) (width 0.2) (layer "F.Cu") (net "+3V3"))
 (segment (start 119.5 137) (end 119.75 137.25) (width 0.2) (layer "F.Cu") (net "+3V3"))
 (segment (start 119.5 136.5) (end 119.5 137) (width 0.2) (layer "F.Cu") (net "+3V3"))
 (segment (start 106.75 131.25) (end 107.5 131.25) (width 0.2) (layer "F.Cu") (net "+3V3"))
 (segment (start 107.5 136) (end 107.5 139.5) (width 0.2) (layer "F.Cu") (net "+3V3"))
 (segment (start 105.5 96.06) (end 105.3875 96.1725) (width 0.2) (layer "F.Cu") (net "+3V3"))
 (segment (start 107.75 133.25) (end 110.3375 133.25) (width 0.2) (layer "F.Cu") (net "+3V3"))
 (segment (start 105.3875 121) (end 108.5 124.1125) (width 0.2) (layer "F.Cu") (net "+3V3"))
 (segment (start 105.3875 96.1725) (end 105.3875 121) (width 0.2) (layer "F.Cu") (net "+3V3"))
 (segment (start 107.75 135.75) (end 110.3375 135.75) (width 0.2) (layer "F.Cu") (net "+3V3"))
 (segment (start 108.25 134.25) (end 110.3375 134.25) (width 0.2) (layer "F.Cu") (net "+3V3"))
 (segment (start 119.5 135.75) (end 119.5 136.5) (width 0.2) (layer "F.Cu") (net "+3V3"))
 (segment (start 121.75 129) (end 124 129) (width 0.2) (layer "F.Cu") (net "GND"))
 (segment (start 111.75 134.75) (end 110.3375 134.75) (width 0.2) (layer "F.Cu") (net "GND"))
 (segment (start 109.4775 112.55) (end 109.4775 124.9775) (width 0.2) (layer "F.Cu") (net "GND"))
 (segment (start 119.75 129.60741) (end 119.75 128.8375) (width 0.2) (layer "F.Cu") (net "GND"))
 (segment (start 117.5 133.5) (end 118.5 134.5) (width 0.2) (layer "F.Cu") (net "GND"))
 (segment (start 109.4775 107.16) (end 112.9825 103.655) (width 0.2) (layer "F.Cu") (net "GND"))
 (segment (start 112.789976 130.75) (end 112.5 130.75) (width 0.2) (layer "F.Cu") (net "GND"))
 (segment (start 106.4375 94.79) (end 107.1675 94.79) (width 0.2) (layer "F.Cu") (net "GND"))
 (segment (start 118.75 130.75) (end 120 130.75) (width 0.2) (layer "F.Cu") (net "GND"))
 (segment (start 117.5 131.5) (end 117.85741 131.5) (width 0.2) (layer "F.Cu") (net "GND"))
 (segment (start 112.5 131.039976) (end 112.5 131.5) (width 0.2) (layer "F.Cu") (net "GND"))
 (segment (start 107.1675 94.79) (end 112.9825 100.605) (width 0.2) (layer "F.Cu") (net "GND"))
 (segment (start 118.678705 130.678705) (end 119.75 129.60741) (width 0.2) (layer "F.Cu") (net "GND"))
 (segment (start 117.5 131.5) (end 117.5 133.5) (width 0.2) (layer "F.Cu") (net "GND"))
 (segment (start 112.5 130.75) (end 111.5 131.75) (width 0.2) (layer "F.Cu") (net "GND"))
 (segment (start 112.5 131.5) (end 117.5 131.5) (width 0.2) (layer "F.Cu") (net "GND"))
 (segment (start 124 129) (end 124 137) (width 0.2) (layer "F.Cu") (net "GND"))
 (segment (start 118.5 134.5) (end 119.25 135.25) (width 0.2) (layer "F.Cu") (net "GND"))
 (segment (start 119.25 135.25) (end 121.6625 135.25) (width 0.2) (layer "F.Cu") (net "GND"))
 (segment (start 120 130.75) (end 121.75 129) (width 0.2) (layer "F.Cu") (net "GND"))
 (segment (start 112.25 132.75) (end 110.3375 132.75) (width 0.2) (layer "F.Cu") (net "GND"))
 (segment (start 109.5 129.5) (end 110 129.5) (width 0.2) (layer "F.Cu") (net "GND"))
 (segment (start 112.5 133) (end 112.25 132.75) (width 0.2) (layer "F.Cu") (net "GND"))
 (segment (start 120 130.75) (end 121.6625 130.75) (width 0.2) (layer "F.Cu") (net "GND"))
 (segment (start 123.9375 94.79) (end 121.8475 94.79) (width 0.2) (layer "F.Cu") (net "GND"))
 (segment (start 118.678705 130.678705) (end 118.75 130.75) (width 0.2) (layer "F.Cu") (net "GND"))
 (segment (start 111.5 131.75) (end 110.3375 131.75) (width 0.2) (layer "F.Cu") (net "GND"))
 (segment (start 110 129.5) (end 110.552606 130.052606) (width 0.2) (layer "F.Cu") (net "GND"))
 (segment (start 112.5 133) (end 112.5 134.5) (width 0.2) (layer "F.Cu") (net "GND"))
 (segment (start 112 135) (end 111.75 135.25) (width 0.2) (layer "F.Cu") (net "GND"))
 (segment (start 117.85741 131.5) (end 118.678705 130.678705) (width 0.2) (layer "F.Cu") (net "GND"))
 (segment (start 124 137) (end 123.75 136.75) (width 0.2) (layer "F.Cu") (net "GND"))
 (segment (start 112.5 131.5) (end 112.5 133) (width 0.2) (layer "F.Cu") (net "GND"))
 (segment (start 121.8475 94.79) (end 116.0325 100.605) (width 0.2) (layer "F.Cu") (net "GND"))
 (segment (start 112.5 134.5) (end 112 135) (width 0.2) (layer "F.Cu") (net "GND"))
 (segment (start 110.552606 130.052606) (end 113.48737 130.052606) (width 0.2) (layer "F.Cu") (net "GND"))
 (segment (start 112.5 130.75) (end 110.3375 130.75) (width 0.2) (layer "F.Cu") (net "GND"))
 (segment (start 123.75 136.75) (end 121.6625 136.75) (width 0.2) (layer "F.Cu") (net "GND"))
 (segment (start 113.48737 130.052606) (end 112.789976 130.75) (width 0.2) (layer "F.Cu") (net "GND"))
 (segment (start 112 135) (end 111.75 134.75) (width 0.2) (layer "F.Cu") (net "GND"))
 (segment (start 111.75 135.25) (end 110.3375 135.25) (width 0.2) (layer "F.Cu") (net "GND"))
 (segment (start 109.4775 112.55) (end 109.4775 107.16) (width 0.2) (layer "F.Cu") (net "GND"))
 (segment (start 109.5 125) (end 109.4775 124.9775) (width 0.2) (layer "F.Cu") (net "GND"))
 (segment (start 112.789976 130.75) (end 112.5 131.039976) (width 0.2) (layer "F.Cu") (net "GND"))
 (via (at 109.4775 124.9775) (size 0.6) (drill 0.3) (layers "F.Cu" "B.Cu") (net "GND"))
 (via (at 109.5 129.5) (size 0.6) (drill 0.3) (layers "F.Cu" "B.Cu") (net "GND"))
 (segment (start 109.4775 124.9775) (end 109.5 125) (width 0.2) (layer "B.Cu") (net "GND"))
 (segment (start 109.5 125) (end 109.5 129.5) (width 0.2) (layer "B.Cu") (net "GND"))
 (segment (start 128 119.31759) (end 121.31759 126) (width 0.2) (layer "F.Cu") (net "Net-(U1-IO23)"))
 (segment (start 123.9375 96.06) (end 128 96.06) (width 0.2) (layer "F.Cu") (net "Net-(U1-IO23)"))
 (segment (start 119.25 128.06759) (end 119.25 128.8375) (width 0.2) (layer "F.Cu") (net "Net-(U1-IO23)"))
 (segment (start 128 96.06) (end 128 119.31759) (width 0.2) (layer "F.Cu") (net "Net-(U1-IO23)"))
 (segment (start 121.31759 126) (end 119.25 128.06759) (width 0.2) (layer "F.Cu") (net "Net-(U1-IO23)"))
 (segment (start 123.9375 106.22) (end 122.9875 106.22) (width 0.2) (layer "F.Cu") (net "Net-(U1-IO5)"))
 (segment (start 122.4575 106.75) (end 122.4575 115.0425) (width 0.2) (layer "F.Cu") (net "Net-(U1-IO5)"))
 (segment (start 116.75 117.25) (end 116.75 128.8375) (width 0.2) (layer "F.Cu") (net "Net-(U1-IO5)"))
 (segment (start 122.9875 106.22) (end 122.4575 106.75) (width 0.2) (layer "F.Cu") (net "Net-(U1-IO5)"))
 (segment (start 117.5 116.5) (end 116.75 117.25) (width 0.2) (layer "F.Cu") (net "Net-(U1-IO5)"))
 (segment (start 121 116.5) (end 117.5 116.5) (width 0.2) (layer "F.Cu") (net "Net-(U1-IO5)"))
 (segment (start 122.4575 115.0425) (end 121 116.5) (width 0.2) (layer "F.Cu") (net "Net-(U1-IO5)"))
 (segment (start 122.0575 113.9425) (end 120.5 115.5) (width 0.2) (layer "F.Cu") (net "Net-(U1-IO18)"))
 (segment (start 123.9375 104.95) (end 122.6075 104.95) (width 0.2) (layer "F.Cu") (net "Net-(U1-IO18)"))
 (segment (start 122.6075 104.95) (end 122.0575 105.5) (width 0.2) (layer "F.Cu") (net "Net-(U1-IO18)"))
 (segment (start 120.5 115.5) (end 117 115.5) (width 0.2) (layer "F.Cu") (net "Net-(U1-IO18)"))
 (segment (start 117 115.5) (end 116.25 116.25) (width 0.2) (layer "F.Cu") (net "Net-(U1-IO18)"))
 (segment (start 116.25 116.25) (end 116.25 128.8375) (width 0.2) (layer "F.Cu") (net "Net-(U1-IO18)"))
 (segment (start 122.0575 105.5) (end 122.0575 113.9425) (width 0.2) (layer "F.Cu") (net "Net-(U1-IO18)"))
 (segment (start 114.75 116.25) (end 114.75 128.8375) (width 0.2) (layer "F.Cu") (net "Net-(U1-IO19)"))
 (segment (start 123.9375 103.68) (end 122.9875 103.68) (width 0.2) (layer "F.Cu") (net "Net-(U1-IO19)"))
 (segment (start 116 115) (end 114.75 116.25) (width 0.2) (layer "F.Cu") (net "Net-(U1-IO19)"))
 (segment (start 121.6575 105.01) (end 121.6575 113.6) (width 0.2) (layer "F.Cu") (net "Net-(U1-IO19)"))
 (segment (start 121.6575 113.6) (end 120.2575 115) (width 0.2) (layer "F.Cu") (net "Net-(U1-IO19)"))
 (segment (start 120.2575 115) (end 116 115) (width 0.2) (layer "F.Cu") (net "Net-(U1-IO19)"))
 (segment (start 122.9875 103.68) (end 121.6575 105.01) (width 0.2) (layer "F.Cu") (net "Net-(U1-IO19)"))
 (segment (start 125.5 121) (end 118.5 121) (width 0.2) (layer "F.Cu") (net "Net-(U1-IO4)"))
 (segment (start 125.5 110.5) (end 125.5 121) (width 0.2) (layer "F.Cu") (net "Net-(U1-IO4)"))
 (segment (start 123.9675 110) (end 125 110) (width 0.2) (layer "F.Cu") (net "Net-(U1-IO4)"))
 (segment (start 123.9375 110.03) (end 123.9675 110) (width 0.2) (layer "F.Cu") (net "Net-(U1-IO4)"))
 (segment (start 113 121) (end 112.75 121.25) (width 0.2) (layer "F.Cu") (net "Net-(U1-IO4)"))
 (segment (start 125 110) (end 125.5 110.5) (width 0.2) (layer "F.Cu") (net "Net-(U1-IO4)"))
 (segment (start 112.75 121.25) (end 112.75 128.8375) (width 0.2) (layer "F.Cu") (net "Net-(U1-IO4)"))
 (via (at 113 121) (size 0.6) (drill 0.3) (layers "F.Cu" "B.Cu") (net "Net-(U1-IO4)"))
 (via (at 118.5 121) (size 0.6) (drill 0.3) (layers "F.Cu" "B.Cu") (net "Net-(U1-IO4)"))
 (segment (start 118.5 121) (end 113 121) (width 0.2) (layer "B.Cu") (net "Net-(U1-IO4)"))
 (segment (start 123.9375 97.33) (end 124 97.3925) (width 0.2) (layer "F.Cu") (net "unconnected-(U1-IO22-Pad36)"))
 (segment (start 124 97.3925) (end 124 97.5) (width 0.2) (layer "F.Cu") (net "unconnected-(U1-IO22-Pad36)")))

